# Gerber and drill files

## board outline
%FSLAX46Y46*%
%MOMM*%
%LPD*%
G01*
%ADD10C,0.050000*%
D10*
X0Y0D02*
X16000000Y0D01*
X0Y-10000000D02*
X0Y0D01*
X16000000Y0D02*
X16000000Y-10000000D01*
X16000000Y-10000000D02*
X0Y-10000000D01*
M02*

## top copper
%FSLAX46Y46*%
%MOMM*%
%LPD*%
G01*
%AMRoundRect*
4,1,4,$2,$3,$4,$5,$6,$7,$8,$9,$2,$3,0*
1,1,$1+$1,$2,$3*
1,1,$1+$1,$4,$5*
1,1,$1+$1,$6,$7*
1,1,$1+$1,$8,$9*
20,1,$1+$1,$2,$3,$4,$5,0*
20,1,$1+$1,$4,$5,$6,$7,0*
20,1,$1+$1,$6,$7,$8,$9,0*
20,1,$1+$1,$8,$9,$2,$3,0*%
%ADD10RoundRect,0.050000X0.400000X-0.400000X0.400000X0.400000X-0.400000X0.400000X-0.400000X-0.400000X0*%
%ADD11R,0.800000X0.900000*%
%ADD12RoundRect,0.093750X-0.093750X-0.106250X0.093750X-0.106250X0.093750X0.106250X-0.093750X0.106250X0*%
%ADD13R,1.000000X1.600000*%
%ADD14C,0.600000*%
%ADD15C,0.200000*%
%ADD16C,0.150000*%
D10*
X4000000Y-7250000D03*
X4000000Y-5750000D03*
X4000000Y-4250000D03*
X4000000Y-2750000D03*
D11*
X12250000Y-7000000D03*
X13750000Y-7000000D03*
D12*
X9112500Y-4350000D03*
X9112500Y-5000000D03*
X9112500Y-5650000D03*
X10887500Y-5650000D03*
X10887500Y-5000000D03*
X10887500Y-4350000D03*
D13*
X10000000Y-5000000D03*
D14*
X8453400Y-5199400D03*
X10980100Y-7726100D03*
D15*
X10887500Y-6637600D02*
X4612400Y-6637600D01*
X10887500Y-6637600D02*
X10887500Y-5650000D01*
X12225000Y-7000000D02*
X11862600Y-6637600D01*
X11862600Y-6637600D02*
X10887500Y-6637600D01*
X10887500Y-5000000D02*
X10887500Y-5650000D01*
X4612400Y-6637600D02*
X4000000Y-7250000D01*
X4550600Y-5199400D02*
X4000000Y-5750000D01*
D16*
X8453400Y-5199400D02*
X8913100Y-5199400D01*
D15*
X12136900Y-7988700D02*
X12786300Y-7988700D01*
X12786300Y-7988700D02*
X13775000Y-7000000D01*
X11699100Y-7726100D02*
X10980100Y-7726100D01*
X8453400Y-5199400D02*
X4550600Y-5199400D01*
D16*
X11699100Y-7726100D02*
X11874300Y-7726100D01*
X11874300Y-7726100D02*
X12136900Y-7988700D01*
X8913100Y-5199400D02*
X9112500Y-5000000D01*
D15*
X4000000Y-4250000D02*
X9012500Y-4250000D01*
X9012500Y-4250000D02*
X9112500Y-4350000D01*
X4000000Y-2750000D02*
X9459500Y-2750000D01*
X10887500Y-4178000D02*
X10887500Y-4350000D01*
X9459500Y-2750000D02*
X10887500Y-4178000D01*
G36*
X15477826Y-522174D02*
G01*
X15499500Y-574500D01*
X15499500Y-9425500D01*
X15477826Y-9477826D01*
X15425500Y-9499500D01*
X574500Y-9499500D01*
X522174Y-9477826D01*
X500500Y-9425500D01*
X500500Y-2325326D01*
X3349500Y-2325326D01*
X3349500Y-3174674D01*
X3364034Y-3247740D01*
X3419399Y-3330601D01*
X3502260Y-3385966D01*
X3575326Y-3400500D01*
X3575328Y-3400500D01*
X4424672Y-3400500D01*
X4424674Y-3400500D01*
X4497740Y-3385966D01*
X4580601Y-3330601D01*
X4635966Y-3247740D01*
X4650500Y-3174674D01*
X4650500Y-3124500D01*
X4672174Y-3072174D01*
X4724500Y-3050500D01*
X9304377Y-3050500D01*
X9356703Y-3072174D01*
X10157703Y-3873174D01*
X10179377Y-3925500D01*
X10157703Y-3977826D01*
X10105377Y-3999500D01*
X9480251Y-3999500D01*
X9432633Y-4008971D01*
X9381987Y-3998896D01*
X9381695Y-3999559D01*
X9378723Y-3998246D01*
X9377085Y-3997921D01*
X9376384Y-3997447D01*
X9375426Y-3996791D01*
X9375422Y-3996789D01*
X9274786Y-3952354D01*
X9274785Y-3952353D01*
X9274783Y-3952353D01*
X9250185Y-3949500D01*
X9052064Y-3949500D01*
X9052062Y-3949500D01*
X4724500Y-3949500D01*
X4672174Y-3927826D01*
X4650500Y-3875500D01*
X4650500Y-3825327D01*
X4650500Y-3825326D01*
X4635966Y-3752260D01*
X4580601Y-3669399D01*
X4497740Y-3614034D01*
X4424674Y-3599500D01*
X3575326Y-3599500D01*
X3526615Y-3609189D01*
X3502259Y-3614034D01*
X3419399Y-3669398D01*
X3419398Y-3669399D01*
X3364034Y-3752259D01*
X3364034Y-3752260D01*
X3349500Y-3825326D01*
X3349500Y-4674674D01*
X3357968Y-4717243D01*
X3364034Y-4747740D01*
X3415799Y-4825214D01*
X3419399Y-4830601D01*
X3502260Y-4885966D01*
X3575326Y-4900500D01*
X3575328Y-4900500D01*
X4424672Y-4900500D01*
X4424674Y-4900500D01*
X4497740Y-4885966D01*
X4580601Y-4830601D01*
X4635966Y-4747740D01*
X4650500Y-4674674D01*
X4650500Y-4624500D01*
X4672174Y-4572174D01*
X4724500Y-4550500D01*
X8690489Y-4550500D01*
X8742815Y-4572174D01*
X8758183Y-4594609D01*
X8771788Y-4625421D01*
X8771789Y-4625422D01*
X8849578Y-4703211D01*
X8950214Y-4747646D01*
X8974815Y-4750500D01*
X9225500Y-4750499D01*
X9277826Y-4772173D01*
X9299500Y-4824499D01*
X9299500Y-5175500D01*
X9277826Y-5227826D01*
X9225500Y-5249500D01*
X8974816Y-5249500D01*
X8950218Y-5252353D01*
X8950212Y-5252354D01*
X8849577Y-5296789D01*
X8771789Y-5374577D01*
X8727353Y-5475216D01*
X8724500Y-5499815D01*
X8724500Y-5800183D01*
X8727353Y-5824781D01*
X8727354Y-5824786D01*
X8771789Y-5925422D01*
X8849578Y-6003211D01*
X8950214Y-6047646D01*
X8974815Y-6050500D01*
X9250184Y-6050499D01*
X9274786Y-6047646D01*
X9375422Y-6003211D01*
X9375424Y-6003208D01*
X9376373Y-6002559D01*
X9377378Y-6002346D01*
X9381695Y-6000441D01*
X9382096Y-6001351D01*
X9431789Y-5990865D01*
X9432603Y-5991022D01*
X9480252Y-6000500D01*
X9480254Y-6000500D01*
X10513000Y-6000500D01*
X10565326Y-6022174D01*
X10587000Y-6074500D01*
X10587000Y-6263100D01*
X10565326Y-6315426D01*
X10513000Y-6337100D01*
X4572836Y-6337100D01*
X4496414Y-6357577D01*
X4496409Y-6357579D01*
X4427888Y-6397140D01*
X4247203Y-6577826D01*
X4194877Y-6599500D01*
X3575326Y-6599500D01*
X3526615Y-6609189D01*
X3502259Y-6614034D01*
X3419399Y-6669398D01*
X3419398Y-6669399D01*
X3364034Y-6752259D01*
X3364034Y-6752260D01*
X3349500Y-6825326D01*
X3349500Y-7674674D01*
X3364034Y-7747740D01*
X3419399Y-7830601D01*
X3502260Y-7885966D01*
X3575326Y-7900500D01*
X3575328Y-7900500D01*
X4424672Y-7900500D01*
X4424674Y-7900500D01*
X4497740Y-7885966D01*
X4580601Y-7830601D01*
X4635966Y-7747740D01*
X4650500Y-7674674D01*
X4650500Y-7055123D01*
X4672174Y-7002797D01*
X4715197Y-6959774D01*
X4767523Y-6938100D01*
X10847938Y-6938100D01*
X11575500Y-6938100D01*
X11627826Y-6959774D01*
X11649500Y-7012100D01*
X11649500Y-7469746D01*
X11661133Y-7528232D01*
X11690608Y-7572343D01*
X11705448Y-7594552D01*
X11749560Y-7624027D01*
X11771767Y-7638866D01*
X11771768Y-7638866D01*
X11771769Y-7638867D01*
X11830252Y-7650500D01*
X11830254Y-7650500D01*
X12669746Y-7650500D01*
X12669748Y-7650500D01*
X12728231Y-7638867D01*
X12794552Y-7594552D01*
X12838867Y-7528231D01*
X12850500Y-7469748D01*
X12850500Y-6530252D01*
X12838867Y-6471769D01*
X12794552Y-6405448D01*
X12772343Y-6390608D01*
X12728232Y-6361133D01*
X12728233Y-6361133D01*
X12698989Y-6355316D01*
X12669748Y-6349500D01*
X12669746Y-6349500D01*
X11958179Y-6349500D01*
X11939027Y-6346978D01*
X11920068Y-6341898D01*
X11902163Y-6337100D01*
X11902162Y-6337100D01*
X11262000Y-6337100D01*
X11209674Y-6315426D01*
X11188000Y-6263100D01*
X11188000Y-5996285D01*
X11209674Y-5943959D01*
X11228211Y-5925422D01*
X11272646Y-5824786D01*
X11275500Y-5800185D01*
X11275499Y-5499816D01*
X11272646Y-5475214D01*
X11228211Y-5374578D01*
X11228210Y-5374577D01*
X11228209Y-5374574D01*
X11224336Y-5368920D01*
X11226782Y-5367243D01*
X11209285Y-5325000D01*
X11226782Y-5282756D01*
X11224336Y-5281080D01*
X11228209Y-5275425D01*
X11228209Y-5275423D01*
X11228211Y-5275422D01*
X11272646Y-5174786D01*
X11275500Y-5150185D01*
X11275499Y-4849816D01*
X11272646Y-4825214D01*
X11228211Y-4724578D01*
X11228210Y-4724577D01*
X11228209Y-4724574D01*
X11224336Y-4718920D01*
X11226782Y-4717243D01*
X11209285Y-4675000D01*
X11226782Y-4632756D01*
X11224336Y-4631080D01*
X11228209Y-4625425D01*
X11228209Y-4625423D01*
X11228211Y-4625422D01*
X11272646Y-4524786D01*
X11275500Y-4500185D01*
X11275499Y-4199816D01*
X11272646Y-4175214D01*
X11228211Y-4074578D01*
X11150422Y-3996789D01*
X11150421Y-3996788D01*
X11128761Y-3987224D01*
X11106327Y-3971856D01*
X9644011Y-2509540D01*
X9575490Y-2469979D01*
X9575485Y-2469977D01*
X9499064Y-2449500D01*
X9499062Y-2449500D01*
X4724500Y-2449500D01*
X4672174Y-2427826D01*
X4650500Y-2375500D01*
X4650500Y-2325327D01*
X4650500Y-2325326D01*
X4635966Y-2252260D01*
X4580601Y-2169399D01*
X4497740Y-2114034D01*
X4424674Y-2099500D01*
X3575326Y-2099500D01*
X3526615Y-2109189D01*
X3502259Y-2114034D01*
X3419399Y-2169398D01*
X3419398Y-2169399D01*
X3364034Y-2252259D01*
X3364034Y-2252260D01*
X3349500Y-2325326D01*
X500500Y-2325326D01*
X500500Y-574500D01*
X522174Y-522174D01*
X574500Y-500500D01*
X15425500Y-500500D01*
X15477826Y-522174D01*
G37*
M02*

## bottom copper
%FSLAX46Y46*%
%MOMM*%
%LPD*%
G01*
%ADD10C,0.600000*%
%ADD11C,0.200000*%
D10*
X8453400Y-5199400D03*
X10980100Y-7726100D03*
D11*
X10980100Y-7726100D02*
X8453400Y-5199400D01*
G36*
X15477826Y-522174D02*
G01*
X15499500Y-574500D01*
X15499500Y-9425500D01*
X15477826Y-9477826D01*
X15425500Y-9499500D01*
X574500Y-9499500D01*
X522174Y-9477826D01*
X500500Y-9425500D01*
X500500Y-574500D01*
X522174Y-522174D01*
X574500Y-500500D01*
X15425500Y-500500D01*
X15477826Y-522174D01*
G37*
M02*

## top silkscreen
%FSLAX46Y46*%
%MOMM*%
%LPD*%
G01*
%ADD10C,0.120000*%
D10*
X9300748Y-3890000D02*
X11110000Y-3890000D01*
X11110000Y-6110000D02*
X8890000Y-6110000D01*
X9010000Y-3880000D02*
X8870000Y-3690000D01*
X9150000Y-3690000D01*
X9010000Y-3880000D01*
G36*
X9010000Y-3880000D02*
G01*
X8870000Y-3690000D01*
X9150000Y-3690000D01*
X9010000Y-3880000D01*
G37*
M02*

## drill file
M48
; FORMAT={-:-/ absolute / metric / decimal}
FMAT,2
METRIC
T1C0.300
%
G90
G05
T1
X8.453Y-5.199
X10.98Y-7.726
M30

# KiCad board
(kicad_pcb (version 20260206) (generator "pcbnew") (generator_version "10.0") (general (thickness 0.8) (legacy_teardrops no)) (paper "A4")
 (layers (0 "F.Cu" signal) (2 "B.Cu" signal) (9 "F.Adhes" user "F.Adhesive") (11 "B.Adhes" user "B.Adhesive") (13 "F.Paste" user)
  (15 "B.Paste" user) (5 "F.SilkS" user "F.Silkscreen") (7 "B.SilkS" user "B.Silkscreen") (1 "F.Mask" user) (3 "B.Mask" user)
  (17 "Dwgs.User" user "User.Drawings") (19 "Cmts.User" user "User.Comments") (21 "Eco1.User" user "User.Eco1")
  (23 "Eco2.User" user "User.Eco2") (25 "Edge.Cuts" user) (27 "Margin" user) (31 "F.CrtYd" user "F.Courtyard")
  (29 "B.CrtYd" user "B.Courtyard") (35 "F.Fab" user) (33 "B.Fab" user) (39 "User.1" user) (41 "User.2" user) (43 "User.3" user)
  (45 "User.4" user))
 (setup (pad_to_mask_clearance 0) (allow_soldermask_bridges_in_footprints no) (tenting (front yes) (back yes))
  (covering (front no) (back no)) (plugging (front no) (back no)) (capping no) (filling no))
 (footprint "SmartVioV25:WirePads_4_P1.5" (layer "F.Cu") (at 4 5 90)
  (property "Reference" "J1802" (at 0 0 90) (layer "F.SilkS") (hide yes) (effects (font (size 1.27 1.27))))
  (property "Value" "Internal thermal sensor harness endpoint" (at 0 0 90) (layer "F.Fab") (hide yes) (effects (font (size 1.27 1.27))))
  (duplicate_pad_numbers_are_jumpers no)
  (pad "1" smd roundrect (at -2.25 0 90) (size 0.9 0.9) (layers "F.Cu" "F.Mask") (roundrect_rratio 0.05555555556) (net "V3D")
   (thermal_bridge_angle 45))
  (pad "2" smd roundrect (at -0.75 0 90) (size 0.9 0.9) (layers "F.Cu" "F.Mask") (roundrect_rratio 0.05555555556) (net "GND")
   (thermal_bridge_angle 45))
  (pad "3" smd roundrect (at 0.75 0 90) (size 0.9 0.9) (layers "F.Cu" "F.Mask") (roundrect_rratio 0.05555555556) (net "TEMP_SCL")
   (thermal_bridge_angle 45))
  (pad "4" smd roundrect (at 2.25 0 90) (size 0.9 0.9) (layers "F.Cu" "F.Mask") (roundrect_rratio 0.05555555556) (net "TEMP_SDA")
   (thermal_bridge_angle 45)))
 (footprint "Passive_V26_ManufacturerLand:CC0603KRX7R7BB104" (layer "F.Cu") (at 13 7)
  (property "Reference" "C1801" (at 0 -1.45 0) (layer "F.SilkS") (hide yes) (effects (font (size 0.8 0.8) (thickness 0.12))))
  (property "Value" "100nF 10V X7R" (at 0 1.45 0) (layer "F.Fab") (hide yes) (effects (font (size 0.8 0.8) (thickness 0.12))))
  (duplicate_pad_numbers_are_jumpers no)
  (pad "1" smd rect (at -0.75 0) (size 0.8 0.9) (layers "F.Cu" "F.Mask" "F.Paste") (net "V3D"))
  (pad "2" smd rect (at 0.75 0) (size 0.8 0.9) (layers "F.Cu" "F.Mask" "F.Paste") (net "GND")))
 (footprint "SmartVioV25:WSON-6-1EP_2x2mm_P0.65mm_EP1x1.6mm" (layer "F.Cu") (at 10 5)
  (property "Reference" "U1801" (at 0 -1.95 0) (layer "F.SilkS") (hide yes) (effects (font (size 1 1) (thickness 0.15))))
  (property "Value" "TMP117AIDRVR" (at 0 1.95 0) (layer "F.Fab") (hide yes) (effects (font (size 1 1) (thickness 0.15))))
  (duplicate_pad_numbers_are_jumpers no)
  (fp_line (start -0.699252 -1.11) (end 1.11 -1.11) (stroke (width 0.12) (type solid)) (layer "F.SilkS"))
  (fp_line (start 1.11 1.11) (end -1.11 1.11) (stroke (width 0.12) (type solid)) (layer "F.SilkS"))
  (fp_poly (pts (xy -0.99 -1.12) (xy -1.13 -1.31) (xy -0.85 -1.31)) (stroke (width 0.12) (type solid)) (fill yes) (layer "F.SilkS"))
  (pad "" smd roundrect (at 0 -0.4) (size 0.81 0.64) (layers "F.Paste") (roundrect_rratio 0.25))
  (pad "" smd roundrect (at 0 0.4) (size 0.81 0.64) (layers "F.Paste") (roundrect_rratio 0.25))
  (pad "1" smd roundrect (at -0.8875 -0.65) (size 0.375 0.4) (layers "F.Cu" "F.Mask" "F.Paste") (roundrect_rratio 0.25) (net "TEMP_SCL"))
  (pad "2" smd roundrect (at -0.8875 0) (size 0.375 0.4) (layers "F.Cu" "F.Mask" "F.Paste") (roundrect_rratio 0.25) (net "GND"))
  (pad "3" smd roundrect (at -0.8875 0.65) (size 0.375 0.4) (layers "F.Cu" "F.Mask" "F.Paste") (roundrect_rratio 0.25))
  (pad "4" smd roundrect (at 0.8875 0.65) (size 0.375 0.4) (layers "F.Cu" "F.Mask" "F.Paste") (roundrect_rratio 0.25) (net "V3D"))
  (pad "5" smd roundrect (at 0.8875 0) (size 0.375 0.4) (layers "F.Cu" "F.Mask" "F.Paste") (roundrect_rratio 0.25) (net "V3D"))
  (pad "6" smd roundrect (at 0.8875 -0.65) (size 0.375 0.4) (layers "F.Cu" "F.Mask" "F.Paste") (roundrect_rratio 0.25) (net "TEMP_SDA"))
  (pad "7" smd rect (at 0 0) (size 1 1.6) (layers "F.Cu" "F.Mask") (zone_connect 2)))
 (gr_line (start 0 0) (end 16 0) (stroke (width 0.05) (type default)) (layer "Edge.Cuts"))
 (gr_line (start 0 10) (end 0 0) (stroke (width 0.05) (type default)) (layer "Edge.Cuts"))
 (gr_line (start 16 0) (end 16 10) (stroke (width 0.05) (type default)) (layer "Edge.Cuts"))
 (gr_line (start 16 10) (end 0 10) (stroke (width 0.05) (type default)) (layer "Edge.Cuts"))
 (segment (start 10.8875 6.6376) (end 4.6124 6.6376) (width 0.2) (layer "F.Cu") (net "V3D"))
 (segment (start 10.8875 6.6376) (end 10.8875 5.65) (width 0.2) (layer "F.Cu") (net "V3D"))
 (segment (start 12.225 7) (end 11.8626 6.6376) (width 0.2) (layer "F.Cu") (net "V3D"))
 (segment (start 11.8626 6.6376) (end 10.8875 6.6376) (width 0.2) (layer "F.Cu") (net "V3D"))
 (segment (start 10.8875 5) (end 10.8875 5.65) (width 0.2) (layer "F.Cu") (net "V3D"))
 (segment (start 4.6124 6.6376) (end 4 7.25) (width 0.2) (layer "F.Cu") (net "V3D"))
 (segment (start 4.5506 5.1994) (end 4 5.75) (width 0.2) (layer "F.Cu") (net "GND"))
 (segment (start 8.4534 5.1994) (end 8.9131 5.1994) (width 0.15) (layer "F.Cu") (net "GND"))
 (segment (start 12.1369 7.9887) (end 12.7863 7.9887) (width 0.2) (layer "F.Cu") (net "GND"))
 (segment (start 12.7863 7.9887) (end 13.775 7) (width 0.2) (layer "F.Cu") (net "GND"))
 (segment (start 11.6991 7.7261) (end 10.9801 7.7261) (width 0.2) (layer "F.Cu") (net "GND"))
 (segment (start 8.4534 5.1994) (end 4.5506 5.1994) (width 0.2) (layer "F.Cu") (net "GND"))
 (segment (start 11.6991 7.7261) (end 11.8743 7.7261) (width 0.15) (layer "F.Cu") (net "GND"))
 (segment (start 11.8743 7.7261) (end 12.1369 7.9887) (width 0.15) (layer "F.Cu") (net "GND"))
 (segment (start 8.9131 5.1994) (end 9.1125 5) (width 0.15) (layer "F.Cu") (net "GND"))
 (via (at 8.4534 5.1994) (size 0.6) (drill 0.3) (layers "F.Cu" "B.Cu") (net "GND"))
 (via (at 10.9801 7.7261) (size 0.6) (drill 0.3) (layers "F.Cu" "B.Cu") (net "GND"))
 (segment (start 10.9801 7.7261) (end 8.4534 5.1994) (width 0.2) (layer "B.Cu") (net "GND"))
 (segment (start 4 4.25) (end 9.0125 4.25) (width 0.2) (layer "F.Cu") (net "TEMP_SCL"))
 (segment (start 9.0125 4.25) (end 9.1125 4.35) (width 0.2) (layer "F.Cu") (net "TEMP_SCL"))
 (segment (start 4 2.75) (end 9.4595 2.75) (width 0.2) (layer "F.Cu") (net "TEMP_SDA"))
 (segment (start 10.8875 4.178) (end 10.8875 4.35) (width 0.2) (layer "F.Cu") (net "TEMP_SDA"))
 (segment (start 9.4595 2.75) (end 10.8875 4.178) (width 0.2) (layer "F.Cu") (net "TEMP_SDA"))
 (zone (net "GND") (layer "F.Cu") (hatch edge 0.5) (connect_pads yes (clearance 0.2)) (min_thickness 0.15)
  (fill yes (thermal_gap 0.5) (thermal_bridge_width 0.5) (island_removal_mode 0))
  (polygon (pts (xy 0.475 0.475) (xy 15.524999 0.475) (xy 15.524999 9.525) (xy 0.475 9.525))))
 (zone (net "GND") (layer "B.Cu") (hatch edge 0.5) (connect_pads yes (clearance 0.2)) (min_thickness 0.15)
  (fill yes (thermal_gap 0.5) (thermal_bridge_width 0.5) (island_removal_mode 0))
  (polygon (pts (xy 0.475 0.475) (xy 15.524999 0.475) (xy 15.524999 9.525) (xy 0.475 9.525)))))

